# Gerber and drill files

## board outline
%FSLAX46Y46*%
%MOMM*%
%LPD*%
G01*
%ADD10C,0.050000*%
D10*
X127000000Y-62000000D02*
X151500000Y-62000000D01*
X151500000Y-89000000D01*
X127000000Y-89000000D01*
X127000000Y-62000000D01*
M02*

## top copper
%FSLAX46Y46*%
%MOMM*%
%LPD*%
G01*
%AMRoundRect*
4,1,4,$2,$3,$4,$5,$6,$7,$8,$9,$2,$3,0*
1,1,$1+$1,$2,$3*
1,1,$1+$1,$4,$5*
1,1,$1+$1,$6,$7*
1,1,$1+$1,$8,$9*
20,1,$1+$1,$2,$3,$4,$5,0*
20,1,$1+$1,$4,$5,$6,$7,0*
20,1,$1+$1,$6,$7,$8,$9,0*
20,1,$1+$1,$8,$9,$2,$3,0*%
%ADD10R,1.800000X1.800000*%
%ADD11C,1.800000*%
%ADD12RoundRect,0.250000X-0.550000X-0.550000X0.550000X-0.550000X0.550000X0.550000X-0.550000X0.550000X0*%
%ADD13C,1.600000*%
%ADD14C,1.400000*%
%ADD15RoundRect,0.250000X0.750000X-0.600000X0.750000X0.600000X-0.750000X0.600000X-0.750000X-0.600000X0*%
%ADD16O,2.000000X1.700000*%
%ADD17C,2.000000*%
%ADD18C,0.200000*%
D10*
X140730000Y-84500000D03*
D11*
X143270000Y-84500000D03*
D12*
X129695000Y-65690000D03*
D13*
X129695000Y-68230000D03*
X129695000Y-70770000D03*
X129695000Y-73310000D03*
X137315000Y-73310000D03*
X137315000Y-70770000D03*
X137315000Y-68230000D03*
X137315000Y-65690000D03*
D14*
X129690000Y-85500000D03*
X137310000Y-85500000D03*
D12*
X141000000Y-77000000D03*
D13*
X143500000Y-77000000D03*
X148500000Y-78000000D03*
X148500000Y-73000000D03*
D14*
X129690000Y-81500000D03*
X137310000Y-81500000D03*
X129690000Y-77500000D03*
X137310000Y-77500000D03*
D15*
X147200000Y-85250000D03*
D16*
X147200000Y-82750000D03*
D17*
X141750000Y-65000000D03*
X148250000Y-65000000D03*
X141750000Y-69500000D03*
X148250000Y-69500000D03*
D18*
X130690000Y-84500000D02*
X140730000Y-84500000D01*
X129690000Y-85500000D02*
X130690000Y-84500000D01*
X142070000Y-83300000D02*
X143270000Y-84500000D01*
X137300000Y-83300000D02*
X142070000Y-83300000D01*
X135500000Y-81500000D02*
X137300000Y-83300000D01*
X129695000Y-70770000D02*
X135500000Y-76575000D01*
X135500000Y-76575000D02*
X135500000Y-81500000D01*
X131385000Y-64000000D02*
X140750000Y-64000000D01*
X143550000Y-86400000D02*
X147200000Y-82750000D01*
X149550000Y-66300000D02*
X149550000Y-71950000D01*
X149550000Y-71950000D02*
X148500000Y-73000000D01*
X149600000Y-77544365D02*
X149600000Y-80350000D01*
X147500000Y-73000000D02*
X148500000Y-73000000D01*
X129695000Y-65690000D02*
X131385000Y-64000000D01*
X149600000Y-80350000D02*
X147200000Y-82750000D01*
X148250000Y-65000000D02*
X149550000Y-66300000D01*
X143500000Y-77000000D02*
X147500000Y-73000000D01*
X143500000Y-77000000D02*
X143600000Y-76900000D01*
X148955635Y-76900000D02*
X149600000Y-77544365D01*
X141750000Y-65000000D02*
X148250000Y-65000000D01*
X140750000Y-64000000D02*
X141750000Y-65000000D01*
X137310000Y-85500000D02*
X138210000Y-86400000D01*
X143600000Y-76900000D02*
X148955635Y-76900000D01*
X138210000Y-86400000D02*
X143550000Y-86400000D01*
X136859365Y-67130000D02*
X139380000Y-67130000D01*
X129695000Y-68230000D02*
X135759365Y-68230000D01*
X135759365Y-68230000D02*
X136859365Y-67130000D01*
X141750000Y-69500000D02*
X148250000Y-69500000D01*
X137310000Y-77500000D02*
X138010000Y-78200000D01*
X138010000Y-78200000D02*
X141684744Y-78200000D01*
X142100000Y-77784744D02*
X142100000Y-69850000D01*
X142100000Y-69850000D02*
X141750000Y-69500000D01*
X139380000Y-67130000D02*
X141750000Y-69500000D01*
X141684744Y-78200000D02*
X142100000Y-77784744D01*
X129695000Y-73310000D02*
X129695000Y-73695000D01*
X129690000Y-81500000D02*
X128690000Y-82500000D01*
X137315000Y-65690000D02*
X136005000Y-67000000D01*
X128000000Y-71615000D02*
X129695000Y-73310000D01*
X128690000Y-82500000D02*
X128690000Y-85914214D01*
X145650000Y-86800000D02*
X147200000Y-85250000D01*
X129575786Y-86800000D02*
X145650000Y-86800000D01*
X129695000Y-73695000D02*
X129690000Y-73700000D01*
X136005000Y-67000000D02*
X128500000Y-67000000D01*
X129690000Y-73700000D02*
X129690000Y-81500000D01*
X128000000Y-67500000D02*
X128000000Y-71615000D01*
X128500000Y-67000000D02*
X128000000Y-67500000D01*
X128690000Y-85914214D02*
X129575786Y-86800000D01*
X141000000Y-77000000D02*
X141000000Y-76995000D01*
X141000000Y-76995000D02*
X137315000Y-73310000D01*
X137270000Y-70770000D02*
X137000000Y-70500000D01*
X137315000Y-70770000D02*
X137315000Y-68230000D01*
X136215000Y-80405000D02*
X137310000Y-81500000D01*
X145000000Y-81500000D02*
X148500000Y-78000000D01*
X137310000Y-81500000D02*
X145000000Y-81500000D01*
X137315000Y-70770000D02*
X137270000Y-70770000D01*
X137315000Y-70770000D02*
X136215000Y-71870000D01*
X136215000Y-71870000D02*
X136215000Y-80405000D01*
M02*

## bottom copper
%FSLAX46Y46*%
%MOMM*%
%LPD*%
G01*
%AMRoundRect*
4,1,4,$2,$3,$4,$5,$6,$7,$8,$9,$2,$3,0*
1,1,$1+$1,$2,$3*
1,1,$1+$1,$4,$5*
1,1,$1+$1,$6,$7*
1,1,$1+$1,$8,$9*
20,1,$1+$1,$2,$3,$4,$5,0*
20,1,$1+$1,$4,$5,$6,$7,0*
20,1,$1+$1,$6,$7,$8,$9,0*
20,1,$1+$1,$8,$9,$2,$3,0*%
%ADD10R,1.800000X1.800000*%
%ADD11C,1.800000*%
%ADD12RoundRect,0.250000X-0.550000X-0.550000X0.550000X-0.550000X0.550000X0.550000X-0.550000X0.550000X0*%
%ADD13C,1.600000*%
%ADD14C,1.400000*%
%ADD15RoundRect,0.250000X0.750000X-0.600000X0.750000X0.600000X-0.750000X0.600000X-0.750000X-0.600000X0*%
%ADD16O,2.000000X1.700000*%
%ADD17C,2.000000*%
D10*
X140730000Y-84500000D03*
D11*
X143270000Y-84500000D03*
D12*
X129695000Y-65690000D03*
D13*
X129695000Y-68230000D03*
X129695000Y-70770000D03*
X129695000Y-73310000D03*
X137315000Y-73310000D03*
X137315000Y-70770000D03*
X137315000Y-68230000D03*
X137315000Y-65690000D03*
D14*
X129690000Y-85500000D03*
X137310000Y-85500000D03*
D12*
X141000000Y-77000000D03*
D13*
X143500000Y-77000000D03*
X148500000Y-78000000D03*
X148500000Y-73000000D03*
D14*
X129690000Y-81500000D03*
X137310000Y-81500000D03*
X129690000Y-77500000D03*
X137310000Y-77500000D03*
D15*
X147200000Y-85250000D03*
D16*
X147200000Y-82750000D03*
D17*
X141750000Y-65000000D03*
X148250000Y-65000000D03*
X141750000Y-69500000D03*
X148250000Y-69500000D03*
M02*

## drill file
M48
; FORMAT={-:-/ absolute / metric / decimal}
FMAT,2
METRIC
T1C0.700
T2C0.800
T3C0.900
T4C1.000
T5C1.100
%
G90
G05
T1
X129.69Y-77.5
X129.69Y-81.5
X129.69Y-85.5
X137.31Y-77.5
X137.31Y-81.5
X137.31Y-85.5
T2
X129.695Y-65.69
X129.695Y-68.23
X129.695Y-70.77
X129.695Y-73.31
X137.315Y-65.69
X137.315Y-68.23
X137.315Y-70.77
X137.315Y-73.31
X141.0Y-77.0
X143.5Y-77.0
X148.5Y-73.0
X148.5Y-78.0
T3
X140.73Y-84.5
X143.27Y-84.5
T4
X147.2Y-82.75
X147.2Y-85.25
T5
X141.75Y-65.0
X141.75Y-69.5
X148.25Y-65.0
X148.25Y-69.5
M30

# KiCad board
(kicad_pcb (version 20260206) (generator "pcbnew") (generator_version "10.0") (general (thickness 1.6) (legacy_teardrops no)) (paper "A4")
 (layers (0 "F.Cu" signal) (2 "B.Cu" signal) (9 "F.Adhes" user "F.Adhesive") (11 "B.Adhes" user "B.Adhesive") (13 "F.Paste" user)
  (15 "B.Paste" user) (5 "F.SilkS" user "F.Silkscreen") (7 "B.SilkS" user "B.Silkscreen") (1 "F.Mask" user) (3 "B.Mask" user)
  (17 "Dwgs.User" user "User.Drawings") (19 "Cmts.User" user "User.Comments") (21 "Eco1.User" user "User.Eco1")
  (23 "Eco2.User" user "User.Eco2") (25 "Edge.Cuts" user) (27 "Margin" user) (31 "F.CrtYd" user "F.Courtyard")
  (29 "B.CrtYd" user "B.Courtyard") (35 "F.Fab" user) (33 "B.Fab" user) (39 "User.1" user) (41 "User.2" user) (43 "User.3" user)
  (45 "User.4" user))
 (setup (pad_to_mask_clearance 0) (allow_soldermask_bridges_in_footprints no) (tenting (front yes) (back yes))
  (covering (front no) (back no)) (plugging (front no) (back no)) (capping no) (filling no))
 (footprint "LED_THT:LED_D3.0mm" (layer "F.Cu") (at 140.73 84.5)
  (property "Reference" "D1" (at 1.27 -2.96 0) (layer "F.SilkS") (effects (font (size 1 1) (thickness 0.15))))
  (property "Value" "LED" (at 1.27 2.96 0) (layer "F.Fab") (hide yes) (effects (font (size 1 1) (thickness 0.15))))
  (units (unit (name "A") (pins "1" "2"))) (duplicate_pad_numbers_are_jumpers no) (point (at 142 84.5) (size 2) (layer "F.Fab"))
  (pad "1" thru_hole rect (at 0 0) (size 1.8 1.8) (drill 0.9) (layers "*.Cu" "*.Mask") (remove_unused_layers no) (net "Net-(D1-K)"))
  (pad "2" thru_hole circle (at 2.54 0) (size 1.8 1.8) (drill 0.9) (layers "*.Cu" "*.Mask") (remove_unused_layers no) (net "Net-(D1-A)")))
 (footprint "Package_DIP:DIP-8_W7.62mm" (layer "F.Cu") (at 129.695 65.69)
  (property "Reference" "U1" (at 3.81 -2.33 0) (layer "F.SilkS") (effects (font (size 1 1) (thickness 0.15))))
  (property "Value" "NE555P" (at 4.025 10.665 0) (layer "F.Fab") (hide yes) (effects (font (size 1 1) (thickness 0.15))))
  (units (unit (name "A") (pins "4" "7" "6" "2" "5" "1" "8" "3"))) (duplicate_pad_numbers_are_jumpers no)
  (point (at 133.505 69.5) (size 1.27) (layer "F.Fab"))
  (pad "1" thru_hole roundrect (at 0 0) (size 1.6 1.6) (drill 0.8) (layers "*.Cu" "*.Mask") (remove_unused_layers no)
   (roundrect_rratio 0.15625) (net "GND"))
  (pad "2" thru_hole circle (at 0 2.54) (size 1.6 1.6) (drill 0.8) (layers "*.Cu" "*.Mask") (remove_unused_layers no) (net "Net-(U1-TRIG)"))
  (pad "3" thru_hole circle (at 0 5.08) (size 1.6 1.6) (drill 0.8) (layers "*.Cu" "*.Mask") (remove_unused_layers no) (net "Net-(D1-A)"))
  (pad "4" thru_hole circle (at 0 7.62) (size 1.6 1.6) (drill 0.8) (layers "*.Cu" "*.Mask") (remove_unused_layers no) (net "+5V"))
  (pad "5" thru_hole circle (at 7.62 7.62) (size 1.6 1.6) (drill 0.8) (layers "*.Cu" "*.Mask") (remove_unused_layers no)
   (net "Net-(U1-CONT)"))
  (pad "6" thru_hole circle (at 7.62 5.08) (size 1.6 1.6) (drill 0.8) (layers "*.Cu" "*.Mask") (remove_unused_layers no)
   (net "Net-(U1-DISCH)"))
  (pad "7" thru_hole circle (at 7.62 2.54) (size 1.6 1.6) (drill 0.8) (layers "*.Cu" "*.Mask") (remove_unused_layers no)
   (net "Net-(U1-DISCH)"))
  (pad "8" thru_hole circle (at 7.62 0) (size 1.6 1.6) (drill 0.8) (layers "*.Cu" "*.Mask") (remove_unused_layers no) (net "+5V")))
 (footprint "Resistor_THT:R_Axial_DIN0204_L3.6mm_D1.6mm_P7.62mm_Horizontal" (layer "F.Cu") (at 129.69 85.5)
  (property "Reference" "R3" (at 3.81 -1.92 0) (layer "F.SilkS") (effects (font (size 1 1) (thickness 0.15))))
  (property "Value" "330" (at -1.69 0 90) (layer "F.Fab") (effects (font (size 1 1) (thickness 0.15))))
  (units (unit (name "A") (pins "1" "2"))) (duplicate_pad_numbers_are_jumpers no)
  (pad "1" thru_hole circle (at 0 0) (size 1.4 1.4) (drill 0.7) (layers "*.Cu" "*.Mask") (remove_unused_layers no) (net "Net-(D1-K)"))
  (pad "2" thru_hole circle (at 7.62 0) (size 1.4 1.4) (drill 0.7) (layers "*.Cu" "*.Mask") (remove_unused_layers no) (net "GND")))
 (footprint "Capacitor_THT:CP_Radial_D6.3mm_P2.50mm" (layer "F.Cu") (at 141 77)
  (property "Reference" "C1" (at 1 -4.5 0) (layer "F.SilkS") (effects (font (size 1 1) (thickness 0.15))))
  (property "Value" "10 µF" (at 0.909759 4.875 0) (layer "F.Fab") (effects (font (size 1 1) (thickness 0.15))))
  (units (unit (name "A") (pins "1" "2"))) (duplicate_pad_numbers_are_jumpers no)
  (pad "1" thru_hole roundrect (at 0 0) (size 1.6 1.6) (drill 0.8) (layers "*.Cu" "*.Mask") (remove_unused_layers no)
   (roundrect_rratio 0.15625) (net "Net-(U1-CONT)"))
  (pad "2" thru_hole circle (at 2.5 0) (size 1.6 1.6) (drill 0.8) (layers "*.Cu" "*.Mask") (remove_unused_layers no) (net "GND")))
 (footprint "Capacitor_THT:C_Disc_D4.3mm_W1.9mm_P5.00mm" (layer "F.Cu") (at 148.5 78 90)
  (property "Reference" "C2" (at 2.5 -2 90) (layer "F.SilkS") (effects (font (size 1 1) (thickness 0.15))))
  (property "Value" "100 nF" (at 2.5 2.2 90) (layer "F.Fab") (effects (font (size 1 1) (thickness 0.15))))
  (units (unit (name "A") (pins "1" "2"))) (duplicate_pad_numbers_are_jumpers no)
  (pad "1" thru_hole circle (at 0 0 90) (size 1.6 1.6) (drill 0.8) (layers "*.Cu" "*.Mask") (remove_unused_layers no) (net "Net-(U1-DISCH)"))
  (pad "2" thru_hole circle (at 5 0 90) (size 1.6 1.6) (drill 0.8) (layers "*.Cu" "*.Mask") (remove_unused_layers no) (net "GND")))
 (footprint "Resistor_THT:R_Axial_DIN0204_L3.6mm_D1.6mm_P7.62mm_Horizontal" (layer "F.Cu") (at 129.69 81.5)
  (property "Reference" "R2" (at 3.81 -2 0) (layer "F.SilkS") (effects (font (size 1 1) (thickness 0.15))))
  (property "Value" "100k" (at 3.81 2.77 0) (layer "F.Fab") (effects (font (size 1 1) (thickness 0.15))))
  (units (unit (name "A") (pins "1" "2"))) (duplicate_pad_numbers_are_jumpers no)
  (pad "1" thru_hole circle (at 0 0) (size 1.4 1.4) (drill 0.7) (layers "*.Cu" "*.Mask") (remove_unused_layers no) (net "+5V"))
  (pad "2" thru_hole circle (at 7.62 0) (size 1.4 1.4) (drill 0.7) (layers "*.Cu" "*.Mask") (remove_unused_layers no) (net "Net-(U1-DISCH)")))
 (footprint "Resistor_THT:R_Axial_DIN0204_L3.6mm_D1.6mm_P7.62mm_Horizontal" (layer "F.Cu") (at 129.69 77.5)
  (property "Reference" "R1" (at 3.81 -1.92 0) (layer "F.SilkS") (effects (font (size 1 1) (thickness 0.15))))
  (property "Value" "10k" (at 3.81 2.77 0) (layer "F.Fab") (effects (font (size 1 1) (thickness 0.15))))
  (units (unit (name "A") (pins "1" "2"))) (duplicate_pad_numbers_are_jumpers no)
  (pad "1" thru_hole circle (at 0 0) (size 1.4 1.4) (drill 0.7) (layers "*.Cu" "*.Mask") (remove_unused_layers no) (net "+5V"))
  (pad "2" thru_hole circle (at 7.62 0) (size 1.4 1.4) (drill 0.7) (layers "*.Cu" "*.Mask") (remove_unused_layers no) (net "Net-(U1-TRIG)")))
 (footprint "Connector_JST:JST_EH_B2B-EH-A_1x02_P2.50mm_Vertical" (layer "F.Cu") (at 147.2 85.25 90)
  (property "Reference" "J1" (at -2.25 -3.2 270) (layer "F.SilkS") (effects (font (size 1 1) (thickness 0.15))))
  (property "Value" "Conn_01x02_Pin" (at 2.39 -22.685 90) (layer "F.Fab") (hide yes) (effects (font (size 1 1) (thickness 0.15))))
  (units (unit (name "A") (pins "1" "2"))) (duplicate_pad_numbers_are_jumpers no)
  (pad "1" thru_hole roundrect (at 0 0 90) (size 1.7 2) (drill 1) (layers "*.Cu" "*.Mask") (remove_unused_layers no)
   (roundrect_rratio 0.147059) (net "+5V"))
  (pad "2" thru_hole oval (at 2.5 0 90) (size 1.7 2) (drill 1) (layers "*.Cu" "*.Mask") (remove_unused_layers no) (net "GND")))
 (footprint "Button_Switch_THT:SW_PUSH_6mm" (layer "F.Cu") (at 141.75 65)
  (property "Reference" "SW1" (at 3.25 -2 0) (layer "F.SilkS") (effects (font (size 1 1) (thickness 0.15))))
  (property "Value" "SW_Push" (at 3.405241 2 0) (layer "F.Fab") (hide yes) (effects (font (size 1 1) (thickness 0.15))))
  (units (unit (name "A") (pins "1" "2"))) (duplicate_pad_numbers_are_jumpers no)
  (pad "1" thru_hole circle (at 0 0 90) (size 2 2) (drill 1.1) (layers "*.Cu" "*.Mask") (remove_unused_layers no) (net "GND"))
  (pad "1" thru_hole circle (at 6.5 0 90) (size 2 2) (drill 1.1) (layers "*.Cu" "*.Mask") (remove_unused_layers no) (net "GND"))
  (pad "2" thru_hole circle (at 0 4.5 90) (size 2 2) (drill 1.1) (layers "*.Cu" "*.Mask") (remove_unused_layers no) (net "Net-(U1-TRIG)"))
  (pad "2" thru_hole circle (at 6.5 4.5 90) (size 2 2) (drill 1.1) (layers "*.Cu" "*.Mask") (remove_unused_layers no) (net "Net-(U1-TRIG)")))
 (gr_rect (start 127 62) (end 151.5 89) (stroke (width 0.05) (type default)) (fill no) (layer "Edge.Cuts"))
 (segment (start 130.69 84.5) (end 140.73 84.5) (width 0.2) (layer "F.Cu") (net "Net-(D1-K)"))
 (segment (start 129.69 85.5) (end 130.69 84.5) (width 0.2) (layer "F.Cu") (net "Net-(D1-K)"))
 (segment (start 142.07 83.3) (end 143.27 84.5) (width 0.2) (layer "F.Cu") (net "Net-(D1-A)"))
 (segment (start 137.3 83.3) (end 142.07 83.3) (width 0.2) (layer "F.Cu") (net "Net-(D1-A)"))
 (segment (start 135.5 81.5) (end 137.3 83.3) (width 0.2) (layer "F.Cu") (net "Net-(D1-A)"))
 (segment (start 129.695 70.77) (end 135.5 76.575) (width 0.2) (layer "F.Cu") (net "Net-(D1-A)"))
 (segment (start 135.5 76.575) (end 135.5 81.5) (width 0.2) (layer "F.Cu") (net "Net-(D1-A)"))
 (segment (start 131.385 64) (end 140.75 64) (width 0.2) (layer "F.Cu") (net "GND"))
 (segment (start 143.55 86.4) (end 147.2 82.75) (width 0.2) (layer "F.Cu") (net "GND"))
 (segment (start 149.55 66.3) (end 149.55 71.95) (width 0.2) (layer "F.Cu") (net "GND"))
 (segment (start 149.55 71.95) (end 148.5 73) (width 0.2) (layer "F.Cu") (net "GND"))
 (segment (start 149.6 77.544365) (end 149.6 80.35) (width 0.2) (layer "F.Cu") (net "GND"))
 (segment (start 147.5 73) (end 148.5 73) (width 0.2) (layer "F.Cu") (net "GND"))
 (segment (start 129.695 65.69) (end 131.385 64) (width 0.2) (layer "F.Cu") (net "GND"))
 (segment (start 149.6 80.35) (end 147.2 82.75) (width 0.2) (layer "F.Cu") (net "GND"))
 (segment (start 148.25 65) (end 149.55 66.3) (width 0.2) (layer "F.Cu") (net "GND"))
 (segment (start 143.5 77) (end 147.5 73) (width 0.2) (layer "F.Cu") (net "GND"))
 (segment (start 143.5 77) (end 143.6 76.9) (width 0.2) (layer "F.Cu") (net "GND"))
 (segment (start 148.955635 76.9) (end 149.6 77.544365) (width 0.2) (layer "F.Cu") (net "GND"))
 (segment (start 141.75 65) (end 148.25 65) (width 0.2) (layer "F.Cu") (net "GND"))
 (segment (start 140.75 64) (end 141.75 65) (width 0.2) (layer "F.Cu") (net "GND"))
 (segment (start 137.31 85.5) (end 138.21 86.4) (width 0.2) (layer "F.Cu") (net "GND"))
 (segment (start 143.6 76.9) (end 148.955635 76.9) (width 0.2) (layer "F.Cu") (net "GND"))
 (segment (start 138.21 86.4) (end 143.55 86.4) (width 0.2) (layer "F.Cu") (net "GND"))
 (segment (start 136.859365 67.13) (end 139.38 67.13) (width 0.2) (layer "F.Cu") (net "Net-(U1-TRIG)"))
 (segment (start 129.695 68.23) (end 135.759365 68.23) (width 0.2) (layer "F.Cu") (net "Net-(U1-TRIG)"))
 (segment (start 135.759365 68.23) (end 136.859365 67.13) (width 0.2) (layer "F.Cu") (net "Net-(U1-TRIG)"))
 (segment (start 141.75 69.5) (end 148.25 69.5) (width 0.2) (layer "F.Cu") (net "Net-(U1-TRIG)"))
 (segment (start 137.31 77.5) (end 138.01 78.2) (width 0.2) (layer "F.Cu") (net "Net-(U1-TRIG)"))
 (segment (start 138.01 78.2) (end 141.684744 78.2) (width 0.2) (layer "F.Cu") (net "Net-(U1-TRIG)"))
 (segment (start 142.1 77.784744) (end 142.1 69.85) (width 0.2) (layer "F.Cu") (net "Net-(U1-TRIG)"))
 (segment (start 142.1 69.85) (end 141.75 69.5) (width 0.2) (layer "F.Cu") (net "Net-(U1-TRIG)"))
 (segment (start 139.38 67.13) (end 141.75 69.5) (width 0.2) (layer "F.Cu") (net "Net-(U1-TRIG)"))
 (segment (start 141.684744 78.2) (end 142.1 77.784744) (width 0.2) (layer "F.Cu") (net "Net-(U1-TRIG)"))
 (segment (start 129.695 73.31) (end 129.695 73.695) (width 0.2) (layer "F.Cu") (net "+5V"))
 (segment (start 129.69 81.5) (end 128.69 82.5) (width 0.2) (layer "F.Cu") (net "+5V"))
 (segment (start 137.315 65.69) (end 136.005 67) (width 0.2) (layer "F.Cu") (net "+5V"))
 (segment (start 128 71.615) (end 129.695 73.31) (width 0.2) (layer "F.Cu") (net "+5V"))
 (segment (start 128.69 82.5) (end 128.69 85.914214) (width 0.2) (layer "F.Cu") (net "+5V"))
 (segment (start 145.65 86.8) (end 147.2 85.25) (width 0.2) (layer "F.Cu") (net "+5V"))
 (segment (start 129.575786 86.8) (end 145.65 86.8) (width 0.2) (layer "F.Cu") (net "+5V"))
 (segment (start 129.695 73.695) (end 129.69 73.7) (width 0.2) (layer "F.Cu") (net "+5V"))
 (segment (start 136.005 67) (end 128.5 67) (width 0.2) (layer "F.Cu") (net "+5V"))
 (segment (start 129.69 73.7) (end 129.69 81.5) (width 0.2) (layer "F.Cu") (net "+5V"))
 (segment (start 128 67.5) (end 128 71.615) (width 0.2) (layer "F.Cu") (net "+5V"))
 (segment (start 128.5 67) (end 128 67.5) (width 0.2) (layer "F.Cu") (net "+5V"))
 (segment (start 128.69 85.914214) (end 129.575786 86.8) (width 0.2) (layer "F.Cu") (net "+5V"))
 (segment (start 141 77) (end 141 76.995) (width 0.2) (layer "F.Cu") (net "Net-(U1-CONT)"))
 (segment (start 141 76.995) (end 137.315 73.31) (width 0.2) (layer "F.Cu") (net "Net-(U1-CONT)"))
 (segment (start 137.27 70.77) (end 137 70.5) (width 0.2) (layer "F.Cu") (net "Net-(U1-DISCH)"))
 (segment (start 137.315 70.77) (end 137.315 68.23) (width 0.2) (layer "F.Cu") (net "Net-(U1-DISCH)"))
 (segment (start 136.215 80.405) (end 137.31 81.5) (width 0.2) (layer "F.Cu") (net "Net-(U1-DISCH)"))
 (segment (start 145 81.5) (end 148.5 78) (width 0.2) (layer "F.Cu") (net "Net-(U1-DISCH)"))
 (segment (start 137.31 81.5) (end 145 81.5) (width 0.2) (layer "F.Cu") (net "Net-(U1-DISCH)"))
 (segment (start 137.315 70.77) (end 137.27 70.77) (width 0.2) (layer "F.Cu") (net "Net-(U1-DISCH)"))
 (segment (start 137.315 70.77) (end 136.215 71.87) (width 0.2) (layer "F.Cu") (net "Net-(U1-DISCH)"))
 (segment (start 136.215 71.87) (end 136.215 80.405) (width 0.2) (layer "F.Cu") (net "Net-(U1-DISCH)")))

